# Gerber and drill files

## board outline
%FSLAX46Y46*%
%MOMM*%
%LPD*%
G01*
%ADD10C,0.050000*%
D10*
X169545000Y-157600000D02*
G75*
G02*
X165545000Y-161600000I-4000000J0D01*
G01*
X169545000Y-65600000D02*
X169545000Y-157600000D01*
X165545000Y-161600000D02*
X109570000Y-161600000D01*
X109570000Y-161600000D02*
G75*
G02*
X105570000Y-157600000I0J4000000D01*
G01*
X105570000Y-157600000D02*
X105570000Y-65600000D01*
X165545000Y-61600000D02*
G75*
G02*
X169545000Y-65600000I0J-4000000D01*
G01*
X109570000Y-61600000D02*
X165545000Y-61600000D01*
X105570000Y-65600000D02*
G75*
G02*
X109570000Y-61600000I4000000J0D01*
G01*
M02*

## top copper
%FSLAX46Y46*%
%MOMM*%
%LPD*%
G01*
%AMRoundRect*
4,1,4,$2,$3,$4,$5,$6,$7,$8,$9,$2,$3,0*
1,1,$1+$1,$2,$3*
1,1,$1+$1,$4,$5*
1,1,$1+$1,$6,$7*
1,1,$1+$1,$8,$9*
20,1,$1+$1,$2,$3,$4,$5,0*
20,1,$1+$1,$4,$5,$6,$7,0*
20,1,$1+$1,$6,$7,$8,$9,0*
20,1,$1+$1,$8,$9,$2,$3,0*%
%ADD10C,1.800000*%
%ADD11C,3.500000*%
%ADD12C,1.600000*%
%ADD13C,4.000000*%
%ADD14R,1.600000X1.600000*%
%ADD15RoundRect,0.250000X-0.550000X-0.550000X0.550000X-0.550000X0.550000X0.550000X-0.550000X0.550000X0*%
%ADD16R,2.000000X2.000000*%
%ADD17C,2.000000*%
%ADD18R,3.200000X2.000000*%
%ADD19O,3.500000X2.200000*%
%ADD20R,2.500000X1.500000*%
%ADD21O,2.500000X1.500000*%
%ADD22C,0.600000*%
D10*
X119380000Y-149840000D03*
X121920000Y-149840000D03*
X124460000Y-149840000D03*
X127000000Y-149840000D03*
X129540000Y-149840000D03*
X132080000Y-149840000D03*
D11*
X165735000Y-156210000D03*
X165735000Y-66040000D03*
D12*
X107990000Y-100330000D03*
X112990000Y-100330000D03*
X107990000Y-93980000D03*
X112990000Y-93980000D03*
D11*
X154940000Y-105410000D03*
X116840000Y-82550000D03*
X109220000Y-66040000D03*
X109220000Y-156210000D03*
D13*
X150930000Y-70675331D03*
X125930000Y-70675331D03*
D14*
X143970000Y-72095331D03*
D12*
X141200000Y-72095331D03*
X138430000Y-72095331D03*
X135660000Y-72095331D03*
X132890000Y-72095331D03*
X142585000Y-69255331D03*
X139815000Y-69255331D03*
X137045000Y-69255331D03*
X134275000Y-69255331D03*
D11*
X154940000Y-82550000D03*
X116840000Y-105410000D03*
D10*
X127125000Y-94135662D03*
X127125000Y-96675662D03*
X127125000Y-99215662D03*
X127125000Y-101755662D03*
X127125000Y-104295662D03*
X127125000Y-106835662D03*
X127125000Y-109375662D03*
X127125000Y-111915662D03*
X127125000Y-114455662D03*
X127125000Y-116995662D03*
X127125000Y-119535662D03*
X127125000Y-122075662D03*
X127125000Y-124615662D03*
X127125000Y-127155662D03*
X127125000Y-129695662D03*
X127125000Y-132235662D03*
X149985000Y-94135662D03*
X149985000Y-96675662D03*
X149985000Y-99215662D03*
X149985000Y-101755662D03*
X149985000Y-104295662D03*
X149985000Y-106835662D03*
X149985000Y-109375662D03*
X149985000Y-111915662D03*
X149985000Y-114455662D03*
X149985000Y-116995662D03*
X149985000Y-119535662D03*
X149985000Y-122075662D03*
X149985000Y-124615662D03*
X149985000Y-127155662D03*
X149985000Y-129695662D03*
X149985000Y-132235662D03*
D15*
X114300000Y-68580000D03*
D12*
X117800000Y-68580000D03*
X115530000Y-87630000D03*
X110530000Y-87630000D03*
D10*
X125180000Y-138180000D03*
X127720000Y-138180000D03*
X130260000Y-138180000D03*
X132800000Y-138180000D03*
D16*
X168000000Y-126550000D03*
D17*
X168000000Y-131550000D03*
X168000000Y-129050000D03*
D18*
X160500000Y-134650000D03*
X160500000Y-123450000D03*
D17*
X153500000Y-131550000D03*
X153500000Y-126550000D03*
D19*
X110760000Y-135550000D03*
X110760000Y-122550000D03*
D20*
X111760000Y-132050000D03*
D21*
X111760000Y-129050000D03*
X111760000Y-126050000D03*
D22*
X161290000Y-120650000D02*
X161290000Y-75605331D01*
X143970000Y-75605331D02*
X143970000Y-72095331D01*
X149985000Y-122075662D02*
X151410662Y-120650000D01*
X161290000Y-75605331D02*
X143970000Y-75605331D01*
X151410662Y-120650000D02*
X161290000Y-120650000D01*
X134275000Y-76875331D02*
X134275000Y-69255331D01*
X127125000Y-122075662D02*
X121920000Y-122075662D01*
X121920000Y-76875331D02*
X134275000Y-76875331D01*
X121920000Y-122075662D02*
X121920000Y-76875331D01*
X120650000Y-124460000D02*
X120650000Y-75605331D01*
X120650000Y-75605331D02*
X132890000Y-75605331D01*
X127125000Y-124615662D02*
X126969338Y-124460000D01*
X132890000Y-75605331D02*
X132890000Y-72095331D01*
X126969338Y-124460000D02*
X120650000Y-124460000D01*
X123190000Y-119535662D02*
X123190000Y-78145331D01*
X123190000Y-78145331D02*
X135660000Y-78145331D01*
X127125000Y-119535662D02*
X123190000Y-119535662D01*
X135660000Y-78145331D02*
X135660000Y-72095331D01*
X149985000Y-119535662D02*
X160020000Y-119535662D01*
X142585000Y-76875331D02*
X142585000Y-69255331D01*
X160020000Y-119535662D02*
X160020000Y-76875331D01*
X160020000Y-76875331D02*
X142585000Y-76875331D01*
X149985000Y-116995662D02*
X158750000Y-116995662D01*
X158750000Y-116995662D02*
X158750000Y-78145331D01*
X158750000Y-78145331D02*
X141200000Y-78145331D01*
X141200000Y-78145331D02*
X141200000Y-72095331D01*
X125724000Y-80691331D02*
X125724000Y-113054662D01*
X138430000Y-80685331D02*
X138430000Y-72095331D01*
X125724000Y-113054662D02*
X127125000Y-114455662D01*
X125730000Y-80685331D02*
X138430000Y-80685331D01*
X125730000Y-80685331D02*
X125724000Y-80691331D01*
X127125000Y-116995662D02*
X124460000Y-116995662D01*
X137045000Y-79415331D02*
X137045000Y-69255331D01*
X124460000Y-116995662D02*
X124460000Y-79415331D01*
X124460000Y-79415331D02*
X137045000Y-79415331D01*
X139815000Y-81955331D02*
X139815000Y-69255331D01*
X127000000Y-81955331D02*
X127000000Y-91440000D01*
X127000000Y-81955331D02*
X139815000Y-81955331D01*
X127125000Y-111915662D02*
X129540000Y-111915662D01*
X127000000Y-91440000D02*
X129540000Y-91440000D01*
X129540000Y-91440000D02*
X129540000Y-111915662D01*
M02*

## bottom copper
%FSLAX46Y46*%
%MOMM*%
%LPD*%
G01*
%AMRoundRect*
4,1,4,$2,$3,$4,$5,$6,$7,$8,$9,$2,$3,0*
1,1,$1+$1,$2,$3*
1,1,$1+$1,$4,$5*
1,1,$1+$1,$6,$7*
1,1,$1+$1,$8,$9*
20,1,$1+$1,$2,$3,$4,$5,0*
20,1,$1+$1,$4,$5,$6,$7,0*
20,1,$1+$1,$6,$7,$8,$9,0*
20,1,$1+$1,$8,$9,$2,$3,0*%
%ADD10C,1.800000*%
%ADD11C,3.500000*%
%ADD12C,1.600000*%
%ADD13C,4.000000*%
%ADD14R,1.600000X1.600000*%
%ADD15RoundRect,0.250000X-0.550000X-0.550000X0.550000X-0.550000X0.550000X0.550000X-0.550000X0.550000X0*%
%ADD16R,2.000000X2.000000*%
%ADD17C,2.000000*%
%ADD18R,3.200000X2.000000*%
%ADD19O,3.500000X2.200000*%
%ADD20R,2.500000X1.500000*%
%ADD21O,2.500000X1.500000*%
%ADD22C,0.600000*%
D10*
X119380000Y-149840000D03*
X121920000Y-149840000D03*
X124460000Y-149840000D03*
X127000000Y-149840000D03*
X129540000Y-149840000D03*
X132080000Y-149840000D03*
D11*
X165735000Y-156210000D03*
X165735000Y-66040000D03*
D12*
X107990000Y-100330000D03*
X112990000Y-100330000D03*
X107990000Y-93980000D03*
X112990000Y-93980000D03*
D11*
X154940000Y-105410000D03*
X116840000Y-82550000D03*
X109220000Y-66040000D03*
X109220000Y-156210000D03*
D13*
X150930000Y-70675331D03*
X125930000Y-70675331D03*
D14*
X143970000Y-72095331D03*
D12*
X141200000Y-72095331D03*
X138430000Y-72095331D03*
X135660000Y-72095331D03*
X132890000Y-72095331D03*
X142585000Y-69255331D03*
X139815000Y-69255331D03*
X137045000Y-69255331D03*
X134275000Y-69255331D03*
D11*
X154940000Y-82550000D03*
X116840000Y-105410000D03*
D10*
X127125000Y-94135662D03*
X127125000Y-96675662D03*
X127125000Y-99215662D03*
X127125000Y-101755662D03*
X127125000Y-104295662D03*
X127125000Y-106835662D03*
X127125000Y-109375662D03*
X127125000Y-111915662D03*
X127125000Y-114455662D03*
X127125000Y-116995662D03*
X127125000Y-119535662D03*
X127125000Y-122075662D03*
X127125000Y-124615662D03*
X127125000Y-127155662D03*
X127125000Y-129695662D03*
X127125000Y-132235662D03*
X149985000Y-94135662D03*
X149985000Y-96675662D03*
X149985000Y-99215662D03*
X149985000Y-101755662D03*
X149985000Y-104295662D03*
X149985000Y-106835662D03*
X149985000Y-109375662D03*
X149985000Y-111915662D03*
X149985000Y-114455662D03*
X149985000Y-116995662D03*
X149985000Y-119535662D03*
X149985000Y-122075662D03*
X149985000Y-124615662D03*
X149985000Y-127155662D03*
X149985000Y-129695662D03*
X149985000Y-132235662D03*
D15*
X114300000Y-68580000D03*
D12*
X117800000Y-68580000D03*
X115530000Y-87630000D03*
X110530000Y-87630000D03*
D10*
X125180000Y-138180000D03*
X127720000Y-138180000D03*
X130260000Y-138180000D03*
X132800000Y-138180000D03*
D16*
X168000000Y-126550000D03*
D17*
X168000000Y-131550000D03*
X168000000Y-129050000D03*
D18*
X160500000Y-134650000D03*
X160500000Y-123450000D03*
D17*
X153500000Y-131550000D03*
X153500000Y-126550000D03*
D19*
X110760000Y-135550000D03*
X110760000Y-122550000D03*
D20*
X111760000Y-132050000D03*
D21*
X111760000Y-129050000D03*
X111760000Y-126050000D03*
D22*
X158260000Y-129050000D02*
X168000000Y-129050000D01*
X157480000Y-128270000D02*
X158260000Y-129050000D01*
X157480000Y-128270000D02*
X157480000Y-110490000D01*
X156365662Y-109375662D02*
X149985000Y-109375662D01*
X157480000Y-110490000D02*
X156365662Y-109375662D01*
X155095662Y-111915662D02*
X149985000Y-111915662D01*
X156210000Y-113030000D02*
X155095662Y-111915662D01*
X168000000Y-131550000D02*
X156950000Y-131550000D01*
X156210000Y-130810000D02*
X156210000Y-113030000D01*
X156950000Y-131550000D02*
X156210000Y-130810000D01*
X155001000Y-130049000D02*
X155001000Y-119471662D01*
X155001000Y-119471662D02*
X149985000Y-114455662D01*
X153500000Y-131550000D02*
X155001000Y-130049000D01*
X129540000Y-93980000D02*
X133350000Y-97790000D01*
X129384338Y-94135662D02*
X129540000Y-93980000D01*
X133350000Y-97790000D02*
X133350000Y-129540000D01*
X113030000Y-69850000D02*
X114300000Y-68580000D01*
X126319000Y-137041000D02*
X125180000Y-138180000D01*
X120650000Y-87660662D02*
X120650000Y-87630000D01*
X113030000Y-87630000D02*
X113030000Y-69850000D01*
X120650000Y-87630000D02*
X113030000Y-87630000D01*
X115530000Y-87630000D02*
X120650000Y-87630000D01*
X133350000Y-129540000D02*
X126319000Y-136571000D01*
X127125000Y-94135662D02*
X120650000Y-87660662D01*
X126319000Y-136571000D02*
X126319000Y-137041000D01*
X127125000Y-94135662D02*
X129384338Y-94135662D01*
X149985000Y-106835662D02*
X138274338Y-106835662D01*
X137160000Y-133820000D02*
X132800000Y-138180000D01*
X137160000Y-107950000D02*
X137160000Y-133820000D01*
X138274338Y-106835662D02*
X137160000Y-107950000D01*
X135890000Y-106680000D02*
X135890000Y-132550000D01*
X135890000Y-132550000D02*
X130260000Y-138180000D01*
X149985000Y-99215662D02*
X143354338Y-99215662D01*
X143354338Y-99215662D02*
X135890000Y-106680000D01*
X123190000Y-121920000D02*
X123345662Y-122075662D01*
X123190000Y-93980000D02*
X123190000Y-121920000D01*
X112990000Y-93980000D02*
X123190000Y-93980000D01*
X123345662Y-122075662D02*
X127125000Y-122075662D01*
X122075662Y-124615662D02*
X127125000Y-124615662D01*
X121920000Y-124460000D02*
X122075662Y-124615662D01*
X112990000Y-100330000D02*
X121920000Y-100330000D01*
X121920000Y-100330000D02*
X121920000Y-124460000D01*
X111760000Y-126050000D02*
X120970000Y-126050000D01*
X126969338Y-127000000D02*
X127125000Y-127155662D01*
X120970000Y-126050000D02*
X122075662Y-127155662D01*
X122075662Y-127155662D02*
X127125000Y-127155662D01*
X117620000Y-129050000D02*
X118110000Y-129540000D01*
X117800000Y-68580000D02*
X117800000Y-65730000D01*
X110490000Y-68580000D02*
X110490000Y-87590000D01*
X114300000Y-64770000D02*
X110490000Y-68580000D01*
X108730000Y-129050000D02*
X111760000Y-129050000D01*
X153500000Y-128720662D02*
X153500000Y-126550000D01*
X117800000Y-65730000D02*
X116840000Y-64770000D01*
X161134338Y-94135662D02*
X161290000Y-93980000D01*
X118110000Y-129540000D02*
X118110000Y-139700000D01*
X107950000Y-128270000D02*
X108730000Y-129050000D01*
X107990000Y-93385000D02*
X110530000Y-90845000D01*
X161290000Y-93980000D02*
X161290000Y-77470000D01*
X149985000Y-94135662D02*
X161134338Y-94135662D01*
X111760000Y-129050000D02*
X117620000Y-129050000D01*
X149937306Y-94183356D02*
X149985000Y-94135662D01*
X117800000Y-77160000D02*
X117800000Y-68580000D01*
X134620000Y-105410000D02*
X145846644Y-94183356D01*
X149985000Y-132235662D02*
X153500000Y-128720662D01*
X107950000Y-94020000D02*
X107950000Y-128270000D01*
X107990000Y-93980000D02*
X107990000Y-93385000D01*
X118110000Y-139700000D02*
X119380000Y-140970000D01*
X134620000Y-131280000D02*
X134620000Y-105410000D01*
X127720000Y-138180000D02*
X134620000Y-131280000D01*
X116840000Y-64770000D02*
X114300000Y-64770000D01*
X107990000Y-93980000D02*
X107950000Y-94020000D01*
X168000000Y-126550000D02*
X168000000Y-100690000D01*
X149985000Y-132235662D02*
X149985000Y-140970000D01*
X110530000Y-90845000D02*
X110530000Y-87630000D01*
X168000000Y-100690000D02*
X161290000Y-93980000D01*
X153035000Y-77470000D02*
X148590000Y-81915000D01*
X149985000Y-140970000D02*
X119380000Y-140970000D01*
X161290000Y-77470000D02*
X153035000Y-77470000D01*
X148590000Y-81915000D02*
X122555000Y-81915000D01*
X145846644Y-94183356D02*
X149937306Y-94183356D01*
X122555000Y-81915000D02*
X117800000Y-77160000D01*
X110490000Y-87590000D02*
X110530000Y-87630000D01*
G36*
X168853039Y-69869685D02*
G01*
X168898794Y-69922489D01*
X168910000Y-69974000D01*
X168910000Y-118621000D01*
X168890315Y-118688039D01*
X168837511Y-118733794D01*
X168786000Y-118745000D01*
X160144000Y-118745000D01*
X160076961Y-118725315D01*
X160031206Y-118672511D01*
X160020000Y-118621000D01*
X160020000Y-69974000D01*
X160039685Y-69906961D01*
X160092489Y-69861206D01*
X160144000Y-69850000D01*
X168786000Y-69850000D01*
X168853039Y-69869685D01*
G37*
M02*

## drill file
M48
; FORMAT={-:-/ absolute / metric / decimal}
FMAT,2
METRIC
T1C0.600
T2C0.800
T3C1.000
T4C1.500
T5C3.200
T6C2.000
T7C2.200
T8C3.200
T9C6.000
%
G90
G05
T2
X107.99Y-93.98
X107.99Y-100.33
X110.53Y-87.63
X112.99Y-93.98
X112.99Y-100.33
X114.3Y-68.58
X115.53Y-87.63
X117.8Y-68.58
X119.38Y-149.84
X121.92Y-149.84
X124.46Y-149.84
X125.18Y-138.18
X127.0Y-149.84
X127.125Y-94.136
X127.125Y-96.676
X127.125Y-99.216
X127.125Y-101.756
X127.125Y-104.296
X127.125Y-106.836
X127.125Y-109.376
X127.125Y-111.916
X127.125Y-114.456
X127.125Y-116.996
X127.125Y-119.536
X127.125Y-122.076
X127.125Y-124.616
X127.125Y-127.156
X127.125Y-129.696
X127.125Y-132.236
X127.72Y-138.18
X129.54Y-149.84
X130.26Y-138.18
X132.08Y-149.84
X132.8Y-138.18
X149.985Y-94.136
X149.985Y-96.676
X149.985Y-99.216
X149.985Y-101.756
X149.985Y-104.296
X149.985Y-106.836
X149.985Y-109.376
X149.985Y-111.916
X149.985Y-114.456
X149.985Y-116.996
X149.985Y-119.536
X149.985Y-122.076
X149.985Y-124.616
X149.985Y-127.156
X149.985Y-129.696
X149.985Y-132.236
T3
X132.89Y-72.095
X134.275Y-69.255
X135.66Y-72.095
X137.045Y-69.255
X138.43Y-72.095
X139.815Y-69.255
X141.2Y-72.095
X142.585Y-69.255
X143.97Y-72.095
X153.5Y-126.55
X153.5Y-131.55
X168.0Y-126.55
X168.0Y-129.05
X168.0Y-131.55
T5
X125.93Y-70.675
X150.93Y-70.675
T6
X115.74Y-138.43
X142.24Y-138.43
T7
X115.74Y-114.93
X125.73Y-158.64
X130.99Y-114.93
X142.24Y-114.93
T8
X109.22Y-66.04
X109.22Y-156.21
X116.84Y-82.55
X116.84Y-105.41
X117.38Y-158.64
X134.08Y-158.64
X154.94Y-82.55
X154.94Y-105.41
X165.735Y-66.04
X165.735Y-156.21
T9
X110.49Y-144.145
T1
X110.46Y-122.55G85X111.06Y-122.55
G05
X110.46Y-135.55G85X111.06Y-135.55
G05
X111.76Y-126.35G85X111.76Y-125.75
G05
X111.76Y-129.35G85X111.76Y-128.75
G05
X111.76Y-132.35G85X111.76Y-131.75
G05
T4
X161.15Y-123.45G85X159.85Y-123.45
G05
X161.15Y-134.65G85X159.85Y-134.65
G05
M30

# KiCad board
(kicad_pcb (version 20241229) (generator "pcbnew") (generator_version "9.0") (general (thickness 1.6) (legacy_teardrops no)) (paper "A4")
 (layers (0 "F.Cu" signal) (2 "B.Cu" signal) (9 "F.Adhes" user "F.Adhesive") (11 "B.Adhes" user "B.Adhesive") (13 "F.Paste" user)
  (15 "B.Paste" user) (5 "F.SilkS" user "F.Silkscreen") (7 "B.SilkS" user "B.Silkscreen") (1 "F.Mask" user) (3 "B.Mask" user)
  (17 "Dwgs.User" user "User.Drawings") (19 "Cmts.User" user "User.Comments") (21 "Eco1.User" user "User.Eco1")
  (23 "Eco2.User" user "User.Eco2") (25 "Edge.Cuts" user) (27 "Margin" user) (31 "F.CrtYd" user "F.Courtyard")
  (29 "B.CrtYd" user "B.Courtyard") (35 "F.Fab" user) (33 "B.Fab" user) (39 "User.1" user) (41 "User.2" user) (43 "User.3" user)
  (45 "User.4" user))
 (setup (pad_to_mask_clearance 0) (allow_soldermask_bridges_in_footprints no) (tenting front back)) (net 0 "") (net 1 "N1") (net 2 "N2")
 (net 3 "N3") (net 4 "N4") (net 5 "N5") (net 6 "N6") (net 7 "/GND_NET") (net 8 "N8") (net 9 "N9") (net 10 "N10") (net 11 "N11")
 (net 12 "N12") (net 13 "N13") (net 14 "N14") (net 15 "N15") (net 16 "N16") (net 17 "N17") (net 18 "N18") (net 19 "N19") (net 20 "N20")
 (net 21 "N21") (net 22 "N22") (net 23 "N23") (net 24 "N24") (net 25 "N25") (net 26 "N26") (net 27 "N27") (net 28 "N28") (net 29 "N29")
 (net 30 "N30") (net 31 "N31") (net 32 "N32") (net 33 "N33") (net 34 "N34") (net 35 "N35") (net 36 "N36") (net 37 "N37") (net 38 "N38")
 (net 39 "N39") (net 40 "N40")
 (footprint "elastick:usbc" (layer "F.Cu") (at 125.73 148.64)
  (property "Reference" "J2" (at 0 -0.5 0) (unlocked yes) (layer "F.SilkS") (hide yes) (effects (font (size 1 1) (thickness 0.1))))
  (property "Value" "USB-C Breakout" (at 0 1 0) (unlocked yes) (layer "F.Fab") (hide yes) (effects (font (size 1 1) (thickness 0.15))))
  (pad "" np_thru_hole circle (at -8.35 10) (size 3.2 3.2) (drill 3.2) (layers "*.Cu" "*.Mask"))
  (pad "" np_thru_hole circle (at 0 10) (size 2.2 2.2) (drill 2.2) (layers "*.Cu" "*.Mask"))
  (pad "" np_thru_hole circle (at 8.35 10) (size 3.2 3.2) (drill 3.2) (layers "*.Cu" "*.Mask"))
  (pad "1" thru_hole circle (at -6.35 1.2) (size 1.8 1.8) (drill 0.8) (layers "*.Cu" "*.Mask") (remove_unused_layers no) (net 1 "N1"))
  (pad "2" thru_hole circle (at -3.81 1.2) (size 1.8 1.8) (drill 0.8) (layers "*.Cu" "*.Mask") (remove_unused_layers no) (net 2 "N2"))
  (pad "3" thru_hole circle (at -1.27 1.2) (size 1.8 1.8) (drill 0.8) (layers "*.Cu" "*.Mask") (remove_unused_layers no) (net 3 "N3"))
  (pad "4" thru_hole circle (at 1.27 1.2) (size 1.8 1.8) (drill 0.8) (layers "*.Cu" "*.Mask") (remove_unused_layers no) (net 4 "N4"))
  (pad "5" thru_hole circle (at 3.81 1.2) (size 1.8 1.8) (drill 0.8) (layers "*.Cu" "*.Mask") (remove_unused_layers no) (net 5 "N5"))
  (pad "6" thru_hole circle (at 6.35 1.2) (size 1.8 1.8) (drill 0.8) (layers "*.Cu" "*.Mask") (remove_unused_layers no) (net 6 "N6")))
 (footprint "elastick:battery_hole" (layer "F.Cu") (at 165.735 156.21)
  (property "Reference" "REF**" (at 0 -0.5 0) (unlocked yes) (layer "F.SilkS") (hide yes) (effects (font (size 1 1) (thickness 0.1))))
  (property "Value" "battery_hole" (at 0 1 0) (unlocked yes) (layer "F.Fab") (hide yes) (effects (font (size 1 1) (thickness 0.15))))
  (pad "" np_thru_hole circle (at 0 0) (size 3.5 3.5) (drill 3.2) (layers "*.Cu" "*.Mask")))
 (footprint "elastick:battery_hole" (layer "F.Cu") (at 165.735 66.04)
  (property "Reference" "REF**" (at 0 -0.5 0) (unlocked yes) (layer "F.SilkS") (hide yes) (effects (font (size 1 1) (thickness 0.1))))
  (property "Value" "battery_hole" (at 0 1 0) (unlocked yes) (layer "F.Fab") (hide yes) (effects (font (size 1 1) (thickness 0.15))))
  (pad "" np_thru_hole circle (at 0 0) (size 3.5 3.5) (drill 3.2) (layers "*.Cu" "*.Mask")))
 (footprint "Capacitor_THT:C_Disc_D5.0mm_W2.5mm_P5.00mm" (layer "F.Cu") (at 107.99 100.33)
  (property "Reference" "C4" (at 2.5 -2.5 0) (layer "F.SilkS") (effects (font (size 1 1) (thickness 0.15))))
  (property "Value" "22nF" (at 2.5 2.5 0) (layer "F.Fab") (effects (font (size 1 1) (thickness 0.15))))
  (pad "1" thru_hole circle (at 0 0) (size 1.6 1.6) (drill 0.8) (layers "*.Cu" "*.Mask") (remove_unused_layers no) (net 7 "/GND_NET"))
  (pad "2" thru_hole circle (at 5 0) (size 1.6 1.6) (drill 0.8) (layers "*.Cu" "*.Mask") (remove_unused_layers no) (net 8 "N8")))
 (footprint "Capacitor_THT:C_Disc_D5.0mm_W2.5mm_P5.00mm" (layer "F.Cu") (at 107.99 93.98)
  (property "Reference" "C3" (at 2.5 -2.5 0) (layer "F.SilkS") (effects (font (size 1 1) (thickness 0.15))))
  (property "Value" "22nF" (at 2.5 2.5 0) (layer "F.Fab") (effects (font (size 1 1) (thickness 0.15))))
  (pad "1" thru_hole circle (at 0 0) (size 1.6 1.6) (drill 0.8) (layers "*.Cu" "*.Mask") (remove_unused_layers no) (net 7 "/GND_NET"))
  (pad "2" thru_hole circle (at 5 0) (size 1.6 1.6) (drill 0.8) (layers "*.Cu" "*.Mask") (remove_unused_layers no) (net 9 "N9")))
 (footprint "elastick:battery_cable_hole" (layer "F.Cu") (at 110.49 144.145)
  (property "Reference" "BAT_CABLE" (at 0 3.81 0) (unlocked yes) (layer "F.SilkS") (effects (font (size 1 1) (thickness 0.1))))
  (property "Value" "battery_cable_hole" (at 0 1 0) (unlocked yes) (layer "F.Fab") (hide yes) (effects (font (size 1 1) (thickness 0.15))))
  (pad "" np_thru_hole circle (at 0 0) (size 6 6) (drill 6) (layers "*.Cu" "*.Mask")))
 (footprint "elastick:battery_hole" (layer "F.Cu") (at 154.94 105.41)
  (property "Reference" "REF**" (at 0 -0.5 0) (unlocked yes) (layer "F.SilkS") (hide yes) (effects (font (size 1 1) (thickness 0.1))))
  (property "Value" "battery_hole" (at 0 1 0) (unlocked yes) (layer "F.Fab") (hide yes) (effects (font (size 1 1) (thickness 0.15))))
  (pad "" np_thru_hole circle (at 0 0) (size 3.5 3.5) (drill 3.2) (layers "*.Cu" "*.Mask")))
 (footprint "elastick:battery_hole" (layer "F.Cu") (at 116.84 82.55)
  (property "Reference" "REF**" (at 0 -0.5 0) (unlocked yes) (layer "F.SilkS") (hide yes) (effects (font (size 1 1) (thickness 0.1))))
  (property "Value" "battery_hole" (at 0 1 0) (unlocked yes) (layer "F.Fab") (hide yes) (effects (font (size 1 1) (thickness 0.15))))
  (pad "" np_thru_hole circle (at 0 0) (size 3.5 3.5) (drill 3.2) (layers "*.Cu" "*.Mask")))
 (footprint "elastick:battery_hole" (layer "F.Cu") (at 109.22 66.04)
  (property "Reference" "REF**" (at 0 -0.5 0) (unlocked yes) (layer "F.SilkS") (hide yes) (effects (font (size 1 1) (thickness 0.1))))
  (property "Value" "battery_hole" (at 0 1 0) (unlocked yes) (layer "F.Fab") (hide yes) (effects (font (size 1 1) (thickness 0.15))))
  (pad "" np_thru_hole circle (at 0 0) (size 3.5 3.5) (drill 3.2) (layers "*.Cu" "*.Mask")))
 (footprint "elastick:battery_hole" (layer "F.Cu") (at 109.22 156.21)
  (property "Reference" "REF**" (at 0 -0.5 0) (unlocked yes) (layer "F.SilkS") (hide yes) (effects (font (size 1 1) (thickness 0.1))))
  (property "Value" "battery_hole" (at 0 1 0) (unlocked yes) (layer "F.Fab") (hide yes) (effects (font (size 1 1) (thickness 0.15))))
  (pad "" np_thru_hole circle (at 0 0) (size 3.5 3.5) (drill 3.2) (layers "*.Cu" "*.Mask")))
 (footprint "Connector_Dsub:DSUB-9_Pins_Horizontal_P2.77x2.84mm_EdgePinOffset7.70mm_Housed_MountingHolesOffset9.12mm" (layer "F.Cu")
  (at 143.97 72.095331 180)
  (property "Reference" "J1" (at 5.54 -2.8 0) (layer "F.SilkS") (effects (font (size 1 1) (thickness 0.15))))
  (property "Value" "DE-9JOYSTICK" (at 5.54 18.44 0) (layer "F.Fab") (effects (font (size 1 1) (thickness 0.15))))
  (pad "0" thru_hole circle (at -6.96 1.42 180) (size 4 4) (drill 3.2) (layers "*.Cu" "*.Mask") (remove_unused_layers no) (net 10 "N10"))
  (pad "0" thru_hole circle (at 18.04 1.42 180) (size 4 4) (drill 3.2) (layers "*.Cu" "*.Mask") (remove_unused_layers no) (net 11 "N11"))
  (pad "1" thru_hole rect (at 0 0 180) (size 1.6 1.6) (drill 1) (layers "*.Cu" "*.Mask") (remove_unused_layers no) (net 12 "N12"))
  (pad "2" thru_hole circle (at 2.77 0 180) (size 1.6 1.6) (drill 1) (layers "*.Cu" "*.Mask") (remove_unused_layers no) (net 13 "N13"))
  (pad "3" thru_hole circle (at 5.54 0 180) (size 1.6 1.6) (drill 1) (layers "*.Cu" "*.Mask") (remove_unused_layers no) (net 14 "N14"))
  (pad "4" thru_hole circle (at 8.31 0 180) (size 1.6 1.6) (drill 1) (layers "*.Cu" "*.Mask") (remove_unused_layers no) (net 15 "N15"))
  (pad "5" thru_hole circle (at 11.08 0 180) (size 1.6 1.6) (drill 1) (layers "*.Cu" "*.Mask") (remove_unused_layers no) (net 8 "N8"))
  (pad "6" thru_hole circle (at 1.385 2.84 180) (size 1.6 1.6) (drill 1) (layers "*.Cu" "*.Mask") (remove_unused_layers no) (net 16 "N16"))
  (pad "7" thru_hole circle (at 4.155 2.84 180) (size 1.6 1.6) (drill 1) (layers "*.Cu" "*.Mask") (remove_unused_layers no) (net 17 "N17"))
  (pad "8" thru_hole circle (at 6.925 2.84 180) (size 1.6 1.6) (drill 1) (layers "*.Cu" "*.Mask") (remove_unused_layers no) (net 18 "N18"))
  (pad "9" thru_hole circle (at 9.695 2.84 180) (size 1.6 1.6) (drill 1) (layers "*.Cu" "*.Mask") (remove_unused_layers no) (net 9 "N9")))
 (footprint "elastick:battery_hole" (layer "F.Cu") (at 154.94 82.55)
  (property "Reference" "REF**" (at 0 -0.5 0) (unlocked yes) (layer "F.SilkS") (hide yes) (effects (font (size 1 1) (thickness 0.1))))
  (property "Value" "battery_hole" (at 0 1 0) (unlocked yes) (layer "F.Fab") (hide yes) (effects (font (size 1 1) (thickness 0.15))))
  (pad "" np_thru_hole circle (at 0 0) (size 3.5 3.5) (drill 3.2) (layers "*.Cu" "*.Mask")))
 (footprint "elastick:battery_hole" (layer "F.Cu") (at 116.84 105.41)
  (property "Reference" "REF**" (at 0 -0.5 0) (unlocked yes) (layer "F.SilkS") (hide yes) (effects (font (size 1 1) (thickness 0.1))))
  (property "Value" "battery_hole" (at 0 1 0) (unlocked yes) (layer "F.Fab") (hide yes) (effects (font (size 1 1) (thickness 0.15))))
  (pad "" np_thru_hole circle (at 0 0) (size 3.5 3.5) (drill 3.2) (layers "*.Cu" "*.Mask")))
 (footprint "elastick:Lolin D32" (layer "F.Cu") (at 134.745 134.775662)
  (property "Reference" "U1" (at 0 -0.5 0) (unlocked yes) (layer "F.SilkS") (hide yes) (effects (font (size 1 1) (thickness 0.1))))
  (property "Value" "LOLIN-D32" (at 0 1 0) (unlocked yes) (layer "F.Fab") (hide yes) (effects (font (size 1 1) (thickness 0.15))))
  (pad "1" thru_hole circle (at -7.62 -40.64) (size 1.8 1.8) (drill 0.8) (layers "*.Cu" "*.Mask") (remove_unused_layers no) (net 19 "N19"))
  (pad "2" thru_hole circle (at -7.62 -38.1) (size 1.8 1.8) (drill 0.8) (layers "*.Cu" "*.Mask") (remove_unused_layers no) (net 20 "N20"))
  (pad "3" thru_hole circle (at -7.62 -35.56) (size 1.8 1.8) (drill 0.8) (layers "*.Cu" "*.Mask") (remove_unused_layers no) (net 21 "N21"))
  (pad "4" thru_hole circle (at -7.62 -33.02) (size 1.8 1.8) (drill 0.8) (layers "*.Cu" "*.Mask") (remove_unused_layers no) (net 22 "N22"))
  (pad "5" thru_hole circle (at -7.62 -30.48) (size 1.8 1.8) (drill 0.8) (layers "*.Cu" "*.Mask") (remove_unused_layers no) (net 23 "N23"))
  (pad "6" thru_hole circle (at -7.62 -27.94) (size 1.8 1.8) (drill 0.8) (layers "*.Cu" "*.Mask") (remove_unused_layers no) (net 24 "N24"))
  (pad "7" thru_hole circle (at -7.62 -25.4) (size 1.8 1.8) (drill 0.8) (layers "*.Cu" "*.Mask") (remove_unused_layers no) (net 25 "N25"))
  (pad "8" thru_hole circle (at -7.62 -22.86) (size 1.8 1.8) (drill 0.8) (layers "*.Cu" "*.Mask") (remove_unused_layers no) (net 17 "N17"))
  (pad "9" thru_hole circle (at -7.62 -20.32) (size 1.8 1.8) (drill 0.8) (layers "*.Cu" "*.Mask") (remove_unused_layers no) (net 14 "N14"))
  (pad "10" thru_hole circle (at -7.62 -17.78) (size 1.8 1.8) (drill 0.8) (layers "*.Cu" "*.Mask") (remove_unused_layers no) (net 18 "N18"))
  (pad "11" thru_hole circle (at -7.62 -15.24) (size 1.8 1.8) (drill 0.8) (layers "*.Cu" "*.Mask") (remove_unused_layers no) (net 15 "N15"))
  (pad "12" thru_hole circle (at -7.62 -12.7) (size 1.8 1.8) (drill 0.8) (layers "*.Cu" "*.Mask") (remove_unused_layers no) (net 9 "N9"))
  (pad "13" thru_hole circle (at -7.62 -10.16) (size 1.8 1.8) (drill 0.8) (layers "*.Cu" "*.Mask") (remove_unused_layers no) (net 8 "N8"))
  (pad "14" thru_hole circle (at -7.62 -7.62) (size 1.8 1.8) (drill 0.8) (layers "*.Cu" "*.Mask") (remove_unused_layers no) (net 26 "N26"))
  (pad "15" thru_hole circle (at -7.62 -5.08) (size 1.8 1.8) (drill 0.8) (layers "*.Cu" "*.Mask") (remove_unused_layers no) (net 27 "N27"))
  (pad "16" thru_hole circle (at -7.62 -2.54) (size 1.8 1.8) (drill 0.8) (layers "*.Cu" "*.Mask") (remove_unused_layers no) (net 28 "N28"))
  (pad "17" thru_hole circle (at 15.24 -40.64) (size 1.8 1.8) (drill 0.8) (layers "*.Cu" "*.Mask") (remove_unused_layers no)
   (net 7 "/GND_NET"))
  (pad "18" thru_hole circle (at 15.24 -38.1) (size 1.8 1.8) (drill 0.8) (layers "*.Cu" "*.Mask") (remove_unused_layers no) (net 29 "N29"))
  (pad "19" thru_hole circle (at 15.24 -35.56) (size 1.8 1.8) (drill 0.8) (layers "*.Cu" "*.Mask") (remove_unused_layers no) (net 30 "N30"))
  (pad "20" thru_hole circle (at 15.24 -33.02) (size 1.8 1.8) (drill 0.8) (layers "*.Cu" "*.Mask") (remove_unused_layers no) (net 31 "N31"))
  (pad "21" thru_hole circle (at 15.24 -30.48) (size 1.8 1.8) (drill 0.8) (layers "*.Cu" "*.Mask") (remove_unused_layers no) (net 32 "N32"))
  (pad "22" thru_hole circle (at 15.24 -27.94) (size 1.8 1.8) (drill 0.8) (layers "*.Cu" "*.Mask") (remove_unused_layers no) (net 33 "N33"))
  (pad "23" thru_hole circle (at 15.24 -25.4) (size 1.8 1.8) (drill 0.8) (layers "*.Cu" "*.Mask") (remove_unused_layers no) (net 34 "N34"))
  (pad "24" thru_hole circle (at 15.24 -22.86) (size 1.8 1.8) (drill 0.8) (layers "*.Cu" "*.Mask") (remove_unused_layers no) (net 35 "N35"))
  (pad "25" thru_hole circle (at 15.24 -20.32) (size 1.8 1.8) (drill 0.8) (layers "*.Cu" "*.Mask") (remove_unused_layers no) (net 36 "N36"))
  (pad "26" thru_hole circle (at 15.24 -17.78) (size 1.8 1.8) (drill 0.8) (layers "*.Cu" "*.Mask") (remove_unused_layers no) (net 13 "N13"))
  (pad "27" thru_hole circle (at 15.24 -15.24) (size 1.8 1.8) (drill 0.8) (layers "*.Cu" "*.Mask") (remove_unused_layers no) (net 16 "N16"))
  (pad "28" thru_hole circle (at 15.24 -12.7) (size 1.8 1.8) (drill 0.8) (layers "*.Cu" "*.Mask") (remove_unused_layers no) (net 12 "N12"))
  (pad "29" thru_hole circle (at 15.24 -10.16) (size 1.8 1.8) (drill 0.8) (layers "*.Cu" "*.Mask") (remove_unused_layers no) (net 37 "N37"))
  (pad "30" thru_hole circle (at 15.24 -7.62) (size 1.8 1.8) (drill 0.8) (layers "*.Cu" "*.Mask") (remove_unused_layers no) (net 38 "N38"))
  (pad "31" thru_hole circle (at 15.24 -5.08) (size 1.8 1.8) (drill 0.8) (layers "*.Cu" "*.Mask") (remove_unused_layers no) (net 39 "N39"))
  (pad "32" thru_hole circle (at 15.24 -2.54) (size 1.8 1.8) (drill 0.8) (layers "*.Cu" "*.Mask") (remove_unused_layers no)
   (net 7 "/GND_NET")))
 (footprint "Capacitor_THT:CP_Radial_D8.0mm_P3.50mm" (layer "F.Cu") (at 114.3 68.58)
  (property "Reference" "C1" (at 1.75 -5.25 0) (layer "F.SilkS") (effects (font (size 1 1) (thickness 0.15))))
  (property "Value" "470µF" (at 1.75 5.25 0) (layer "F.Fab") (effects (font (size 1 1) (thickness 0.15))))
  (pad "1" thru_hole roundrect (at 0 0) (size 1.6 1.6) (drill 0.8) (layers "*.Cu" "*.Mask") (remove_unused_layers no)
   (roundrect_rratio 0.15625) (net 19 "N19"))
  (pad "2" thru_hole circle (at 3.5 0) (size 1.6 1.6) (drill 0.8) (layers "*.Cu" "*.Mask") (remove_unused_layers no) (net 7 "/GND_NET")))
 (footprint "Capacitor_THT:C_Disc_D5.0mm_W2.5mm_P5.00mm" (layer "F.Cu") (at 115.53 87.63 180)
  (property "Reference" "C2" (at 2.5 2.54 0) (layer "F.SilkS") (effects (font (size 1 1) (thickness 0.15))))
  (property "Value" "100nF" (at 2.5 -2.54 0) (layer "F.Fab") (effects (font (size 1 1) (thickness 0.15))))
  (pad "1" thru_hole circle (at 0 0 180) (size 1.6 1.6) (drill 0.8) (layers "*.Cu" "*.Mask") (remove_unused_layers no) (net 19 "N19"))
  (pad "2" thru_hole circle (at 5 0 180) (size 1.6 1.6) (drill 0.8) (layers "*.Cu" "*.Mask") (remove_unused_layers no) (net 7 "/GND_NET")))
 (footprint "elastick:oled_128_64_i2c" (layer "B.Cu") (at 128.99 138.18)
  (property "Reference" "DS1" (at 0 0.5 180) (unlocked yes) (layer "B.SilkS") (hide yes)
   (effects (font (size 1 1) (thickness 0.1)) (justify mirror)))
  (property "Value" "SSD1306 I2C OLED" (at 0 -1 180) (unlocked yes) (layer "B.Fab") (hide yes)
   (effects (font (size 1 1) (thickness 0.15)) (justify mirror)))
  (pad "" np_thru_hole circle (at -13.25 -23.25) (size 2.2 2.2) (drill 2.2) (layers "*.Cu" "*.Mask"))
  (pad "" np_thru_hole circle (at -13.25 0.25) (size 2 2) (drill 2) (layers "*.Cu" "*.Mask"))
  (pad "" np_thru_hole circle (at 2 -23.25) (size 2.2 2.2) (drill 2.2) (layers "*.Cu" "*.Mask"))
  (pad "" np_thru_hole circle (at 13.25 -23.25) (size 2.2 2.2) (drill 2.2) (layers "*.Cu" "*.Mask"))
  (pad "" np_thru_hole circle (at 13.25 0.25) (size 2 2) (drill 2) (layers "*.Cu" "*.Mask"))
  (pad "1" thru_hole circle (at -3.81 0) (size 1.8 1.8) (drill 0.8) (layers "*.Cu" "*.Mask") (remove_unused_layers no) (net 19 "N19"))
  (pad "2" thru_hole circle (at -1.27 0) (size 1.8 1.8) (drill 0.8) (layers "*.Cu" "*.Mask") (remove_unused_layers no) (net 7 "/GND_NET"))
  (pad "3" thru_hole circle (at 1.27 0) (size 1.8 1.8) (drill 0.8) (layers "*.Cu" "*.Mask") (remove_unused_layers no) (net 30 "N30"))
  (pad "4" thru_hole circle (at 3.81 0) (size 1.8 1.8) (drill 0.8) (layers "*.Cu" "*.Mask") (remove_unused_layers no) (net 33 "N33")))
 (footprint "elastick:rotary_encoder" (layer "B.Cu") (at 168 126.55 180)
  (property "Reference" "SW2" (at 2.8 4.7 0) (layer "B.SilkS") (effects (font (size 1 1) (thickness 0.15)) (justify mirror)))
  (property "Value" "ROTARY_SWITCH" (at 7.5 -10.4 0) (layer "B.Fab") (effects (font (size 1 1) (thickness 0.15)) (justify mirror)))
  (pad "A" thru_hole rect (at 0 0 180) (size 2 2) (drill 1) (layers "*.Cu" "*.Mask") (remove_unused_layers no) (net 7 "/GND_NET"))
  (pad "B" thru_hole circle (at 0 -5 180) (size 2 2) (drill 1) (layers "*.Cu" "*.Mask") (remove_unused_layers no) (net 35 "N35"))
  (pad "C" thru_hole circle (at 0 -2.5 180) (size 2 2) (drill 1) (layers "*.Cu" "*.Mask") (remove_unused_layers no) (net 34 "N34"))
  (pad "MP" thru_hole rect (at 7.5 -8.1 180) (size 3.2 2) (drill oval 2.8 1.5) (layers "*.Cu" "*.Mask") (remove_unused_layers no))
  (pad "MP" thru_hole rect (at 7.5 3.1 180) (size 3.2 2) (drill oval 2.8 1.5) (layers "*.Cu" "*.Mask") (remove_unused_layers no))
  (pad "S1" thru_hole circle (at 14.5 -5 180) (size 2 2) (drill 1) (layers "*.Cu" "*.Mask") (remove_unused_layers no) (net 36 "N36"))
  (pad "S2" thru_hole circle (at 14.5 0 180) (size 2 2) (drill 1) (layers "*.Cu" "*.Mask") (remove_unused_layers no) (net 7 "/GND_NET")))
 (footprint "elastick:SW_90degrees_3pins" (layer "B.Cu") (at 111.76 132.05 90)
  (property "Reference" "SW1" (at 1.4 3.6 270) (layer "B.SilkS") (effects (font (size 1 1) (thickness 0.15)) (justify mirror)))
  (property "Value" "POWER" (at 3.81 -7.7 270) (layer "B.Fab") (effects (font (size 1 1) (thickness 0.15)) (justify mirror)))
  (pad "" thru_hole oval (at -3.5 -1 90) (size 2.2 3.5) (drill oval 0.6 1.2) (layers "*.Cu" "*.Mask") (remove_unused_layers no))
  (pad "" thru_hole oval (at 9.5 -1 90) (size 2.2 3.5) (drill oval 0.6 1.2) (layers "*.Cu" "*.Mask") (remove_unused_layers no))
  (pad "1" thru_hole rect (at 0 0 90) (size 1.5 2.5) (drill oval 1.2 0.6) (layers "*.Cu" "*.Mask") (remove_unused_layers no) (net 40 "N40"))
  (pad "2" thru_hole oval (at 3 0 90) (size 1.5 2.5) (drill oval 1.2 0.6) (layers "*.Cu" "*.Mask") (remove_unused_layers no)
   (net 7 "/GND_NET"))
  (pad "3" thru_hole oval (at 6 0 90) (size 1.5 2.5) (drill oval 1.2 0.6) (layers "*.Cu" "*.Mask") (remove_unused_layers no) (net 26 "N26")))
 (gr_arc (start 169.545 157.6) (mid 168.373427 160.428427) (end 165.545 161.6) (stroke (width 0.05) (type default)) (layer "Edge.Cuts"))
 (gr_line (start 169.545 65.6) (end 169.545 157.6) (stroke (width 0.05) (type default)) (layer "Edge.Cuts"))
 (gr_line (start 165.545 161.6) (end 109.57 161.6) (stroke (width 0.05) (type default)) (layer "Edge.Cuts"))
 (gr_arc (start 109.57 161.6) (mid 106.741573 160.428427) (end 105.57 157.6) (stroke (width 0.05) (type default)) (layer "Edge.Cuts"))
 (gr_line (start 105.57 157.6) (end 105.57 65.6) (stroke (width 0.05) (type default)) (layer "Edge.Cuts"))
 (gr_arc (start 165.545 61.6) (mid 168.373427 62.771573) (end 169.545 65.6) (stroke (width 0.05) (type default)) (layer "Edge.Cuts"))
 (gr_line (start 109.57 61.6) (end 165.545 61.6) (stroke (width 0.05) (type default)) (layer "Edge.Cuts"))
 (gr_arc (start 105.57 65.6) (mid 106.741573 62.771573) (end 109.57 61.6) (stroke (width 0.05) (type default)) (layer "Edge.Cuts"))
 (segment (start 158.26 129.05) (end 168 129.05) (width 0.6) (layer "B.Cu") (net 34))
 (segment (start 157.48 128.27) (end 158.26 129.05) (width 0.6) (layer "B.Cu") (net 34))
 (segment (start 157.48 128.27) (end 157.48 110.49) (width 0.6) (layer "B.Cu") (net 34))
 (segment (start 156.365662 109.375662) (end 149.985 109.375662) (width 0.6) (layer "B.Cu") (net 34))
 (segment (start 157.48 110.49) (end 156.365662 109.375662) (width 0.6) (layer "B.Cu") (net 34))
 (segment (start 155.095662 111.915662) (end 149.985 111.915662) (width 0.6) (layer "B.Cu") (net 35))
 (segment (start 156.21 113.03) (end 155.095662 111.915662) (width 0.6) (layer "B.Cu") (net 35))
 (segment (start 168 131.55) (end 156.95 131.55) (width 0.6) (layer "B.Cu") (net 35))
 (segment (start 156.21 130.81) (end 156.21 113.03) (width 0.6) (layer "B.Cu") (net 35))
 (segment (start 156.95 131.55) (end 156.21 130.81) (width 0.6) (layer "B.Cu") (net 35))
 (segment (start 155.001 130.049) (end 155.001 119.471662) (width 0.6) (layer "B.Cu") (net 36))
 (segment (start 155.001 119.471662) (end 149.985 114.455662) (width 0.6) (layer "B.Cu") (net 36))
 (segment (start 153.5 131.55) (end 155.001 130.049) (width 0.6) (layer "B.Cu") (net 36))
 (segment (start 129.54 93.98) (end 133.35 97.79) (width 0.6) (layer "B.Cu") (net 19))
 (segment (start 129.384338 94.135662) (end 129.54 93.98) (width 0.6) (layer "B.Cu") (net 19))
 (segment (start 133.35 97.79) (end 133.35 129.54) (width 0.6) (layer "B.Cu") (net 19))
 (segment (start 113.03 69.85) (end 114.3 68.58) (width 0.6) (layer "B.Cu") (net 19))
 (segment (start 126.319 137.041) (end 125.18 138.18) (width 0.6) (layer "B.Cu") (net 19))
 (segment (start 120.65 87.660662) (end 120.65 87.63) (width 0.6) (layer "B.Cu") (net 19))
 (segment (start 113.03 87.63) (end 113.03 69.85) (width 0.6) (layer "B.Cu") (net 19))
 (segment (start 120.65 87.63) (end 113.03 87.63) (width 0.6) (layer "B.Cu") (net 19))
 (segment (start 115.53 87.63) (end 120.65 87.63) (width 0.6) (layer "B.Cu") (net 19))
 (segment (start 133.35 129.54) (end 126.319 136.571) (width 0.6) (layer "B.Cu") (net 19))
 (segment (start 127.125 94.135662) (end 120.65 87.660662) (width 0.6) (layer "B.Cu") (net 19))
 (segment (start 126.319 136.571) (end 126.319 137.041) (width 0.6) (layer "B.Cu") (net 19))
 (segment (start 127.125 94.135662) (end 129.384338 94.135662) (width 0.6) (layer "B.Cu") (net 19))
 (segment (start 149.985 106.835662) (end 138.274338 106.835662) (width 0.6) (layer "B.Cu") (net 33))
 (segment (start 137.16 133.82) (end 132.8 138.18) (width 0.6) (layer "B.Cu") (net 33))
 (segment (start 137.16 107.95) (end 137.16 133.82) (width 0.6) (layer "B.Cu") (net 33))
 (segment (start 138.274338 106.835662) (end 137.16 107.95) (width 0.6) (layer "B.Cu") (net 33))
 (segment (start 135.89 106.68) (end 135.89 132.55) (width 0.6) (layer "B.Cu") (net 30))
 (segment (start 135.89 132.55) (end 130.26 138.18) (width 0.6) (layer "B.Cu") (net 30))
 (segment (start 149.985 99.215662) (end 143.354338 99.215662) (width 0.6) (layer "B.Cu") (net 30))
 (segment (start 143.354338 99.215662) (end 135.89 106.68) (width 0.6) (layer "B.Cu") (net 30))
 (segment (start 161.29 120.65) (end 161.29 75.605331) (width 0.6) (layer "F.Cu") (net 12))
 (segment (start 143.97 75.605331) (end 143.97 72.095331) (width 0.6) (layer "F.Cu") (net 12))
 (segment (start 149.985 122.075662) (end 151.410662 120.65) (width 0.6) (layer "F.Cu") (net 12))
 (segment (start 161.29 75.605331) (end 143.97 75.605331) (width 0.6) (layer "F.Cu") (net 12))
 (segment (start 151.410662 120.65) (end 161.29 120.65) (width 0.6) (layer "F.Cu") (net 12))
 (segment (start 134.275 76.875331) (end 134.275 69.255331) (width 0.6) (layer "F.Cu") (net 9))
 (segment (start 127.125 122.075662) (end 121.92 122.075662) (width 0.6) (layer "F.Cu") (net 9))
 (segment (start 121.92 76.875331) (end 134.275 76.875331) (width 0.6) (layer "F.Cu") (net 9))
 (segment (start 121.92 122.075662) (end 121.92 76.875331) (width 0.6) (layer "F.Cu") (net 9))
 (segment (start 123.19 121.92) (end 123.345662 122.075662) (width 0.6) (layer "B.Cu") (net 9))
 (segment (start 123.19 93.98) (end 123.19 121.92) (width 0.6) (layer "B.Cu") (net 9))
 (segment (start 112.99 93.98) (end 123.19 93.98) (width 0.6) (layer "B.Cu") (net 9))
 (segment (start 123.345662 122.075662) (end 127.125 122.075662) (width 0.6) (layer "B.Cu") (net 9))
 (segment (start 120.65 124.46) (end 120.65 75.605331) (width 0.6) (layer "F.Cu") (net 8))
 (segment (start 120.65 75.605331) (end 132.89 75.605331) (width 0.6) (layer "F.Cu") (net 8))
 (segment (start 127.125 124.615662) (end 126.969338 124.46) (width 0.6) (layer "F.Cu") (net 8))
 (segment (start 132.89 75.605331) (end 132.89 72.095331) (width 0.6) (layer "F.Cu") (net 8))
 (segment (start 126.969338 124.46) (end 120.65 124.46) (width 0.6) (layer "F.Cu") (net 8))
 (segment (start 122.075662 124.615662) (end 127.125 124.615662) (width 0.6) (layer "B.Cu") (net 8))
 (segment (start 121.92 124.46) (end 122.075662 124.615662) (width 0.6) (layer "B.Cu") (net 8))
 (segment (start 112.99 100.33) (end 121.92 100.33) (width 0.6) (layer "B.Cu") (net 8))
 (segment (start 121.92 100.33) (end 121.92 124.46) (width 0.6) (layer "B.Cu") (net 8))
 (segment (start 123.19 119.535662) (end 123.19 78.145331) (width 0.6) (layer "F.Cu") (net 15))
 (segment (start 123.19 78.145331) (end 135.66 78.145331) (width 0.6) (layer "F.Cu") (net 15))
 (segment (start 127.125 119.535662) (end 123.19 119.535662) (width 0.6) (layer "F.Cu") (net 15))
 (segment (start 135.66 78.145331) (end 135.66 72.095331) (width 0.6) (layer "F.Cu") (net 15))
 (segment (start 149.985 119.535662) (end 160.02 119.535662) (width 0.6) (layer "F.Cu") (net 16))
 (segment (start 142.585 76.875331) (end 142.585 69.255331) (width 0.6) (layer "F.Cu") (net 16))
 (segment (start 160.02 119.535662) (end 160.02 76.875331) (width 0.6) (layer "F.Cu") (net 16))
 (segment (start 160.02 76.875331) (end 142.585 76.875331) (width 0.6) (layer "F.Cu") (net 16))
 (segment (start 149.985 116.995662) (end 158.75 116.995662) (width 0.6) (layer "F.Cu") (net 13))
 (segment (start 158.75 116.995662) (end 158.75 78.145331) (width 0.6) (layer "F.Cu") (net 13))
 (segment (start 158.75 78.145331) (end 141.2 78.145331) (width 0.6) (layer "F.Cu") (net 13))
 (segment (start 141.2 78.145331) (end 141.2 72.095331) (width 0.6) (layer "F.Cu") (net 13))
 (segment (start 125.724 80.691331) (end 125.724 113.054662) (width 0.6) (layer "F.Cu") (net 14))
 (segment (start 138.43 80.685331) (end 138.43 72.095331) (width 0.6) (layer "F.Cu") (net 14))
 (segment (start 125.724 113.054662) (end 127.125 114.455662) (width 0.6) (layer "F.Cu") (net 14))
 (segment (start 125.73 80.685331) (end 138.43 80.685331) (width 0.6) (layer "F.Cu") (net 14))
 (segment (start 125.73 80.685331) (end 125.724 80.691331) (width 0.6) (layer "F.Cu") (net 14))
 (segment (start 127.125 116.995662) (end 124.46 116.995662) (width 0.6) (layer "F.Cu") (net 18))
 (segment (start 137.045 79.415331) (end 137.045 69.255331) (width 0.6) (layer "F.Cu") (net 18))
 (segment (start 124.46 116.995662) (end 124.46 79.415331) (width 0.6) (layer "F.Cu") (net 18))
 (segment (start 124.46 79.415331) (end 137.045 79.415331) (width 0.6) (layer "F.Cu") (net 18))
 (segment (start 139.815 81.955331) (end 139.815 69.255331) (width 0.6) (layer "F.Cu") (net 17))
 (segment (start 127 81.955331) (end 127 91.44) (width 0.6) (layer "F.Cu") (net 17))
 (segment (start 127 81.955331) (end 139.815 81.955331) (width 0.6) (layer "F.Cu") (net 17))
 (segment (start 127.125 111.915662) (end 129.54 111.915662) (width 0.6) (layer "F.Cu") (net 17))
 (segment (start 127 91.44) (end 129.54 91.44) (width 0.6) (layer "F.Cu") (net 17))
 (segment (start 129.54 91.44) (end 129.54 111.915662) (width 0.6) (layer "F.Cu") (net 17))
 (segment (start 111.76 126.05) (end 120.97 126.05) (width 0.6) (layer "B.Cu") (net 26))
 (segment (start 126.969338 127) (end 127.125 127.155662) (width 0.6) (layer "B.Cu") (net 26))
 (segment (start 120.97 126.05) (end 122.075662 127.155662) (width 0.6) (layer "B.Cu") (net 26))
 (segment (start 122.075662 127.155662) (end 127.125 127.155662) (width 0.6) (layer "B.Cu") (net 26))
 (segment (start 117.62 129.05) (end 118.11 129.54) (width 0.6) (layer "B.Cu") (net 7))
 (segment (start 117.8 68.58) (end 117.8 65.73) (width 0.6) (layer "B.Cu") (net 7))
 (segment (start 110.49 68.58) (end 110.49 87.59) (width 0.6) (layer "B.Cu") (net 7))
 (segment (start 114.3 64.77) (end 110.49 68.58) (width 0.6) (layer "B.Cu") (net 7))
 (segment (start 108.73 129.05) (end 111.76 129.05) (width 0.6) (layer "B.Cu") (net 7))
 (segment (start 153.5 128.720662) (end 153.5 126.55) (width 0.6) (layer "B.Cu") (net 7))
 (segment (start 117.8 65.73) (end 116.84 64.77) (width 0.6) (layer "B.Cu") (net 7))
 (segment (start 161.134338 94.135662) (end 161.29 93.98) (width 0.6) (layer "B.Cu") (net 7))
 (segment (start 118.11 129.54) (end 118.11 139.7) (width 0.6) (layer "B.Cu") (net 7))
 (segment (start 107.95 128.27) (end 108.73 129.05) (width 0.6) (layer "B.Cu") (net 7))
 (segment (start 107.99 93.385) (end 110.53 90.845) (width 0.6) (layer "B.Cu") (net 7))
 (segment (start 161.29 93.98) (end 161.29 77.47) (width 0.6) (layer "B.Cu") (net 7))
 (segment (start 149.985 94.135662) (end 161.134338 94.135662) (width 0.6) (layer "B.Cu") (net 7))
 (segment (start 111.76 129.05) (end 117.62 129.05) (width 0.6) (layer "B.Cu") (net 7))
 (segment (start 149.937306 94.183356) (end 149.985 94.135662) (width 0.6) (layer "B.Cu") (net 7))
 (segment (start 117.8 77.16) (end 117.8 68.58) (width 0.6) (layer "B.Cu") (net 7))
 (segment (start 134.62 105.41) (end 145.846644 94.183356) (width 0.6) (layer "B.Cu") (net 7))
 (segment (start 149.985 132.235662) (end 153.5 128.720662) (width 0.6) (layer "B.Cu") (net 7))
 (segment (start 107.95 94.02) (end 107.95 128.27) (width 0.6) (layer "B.Cu") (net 7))
 (segment (start 107.99 93.98) (end 107.99 93.385) (width 0.6) (layer "B.Cu") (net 7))
 (segment (start 118.11 139.7) (end 119.38 140.97) (width 0.6) (layer "B.Cu") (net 7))
 (segment (start 134.62 131.28) (end 134.62 105.41) (width 0.6) (layer "B.Cu") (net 7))
 (segment (start 127.72 138.18) (end 134.62 131.28) (width 0.6) (layer "B.Cu") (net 7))
 (segment (start 116.84 64.77) (end 114.3 64.77) (width 0.6) (layer "B.Cu") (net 7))
 (segment (start 107.99 93.98) (end 107.95 94.02) (width 0.6) (layer "B.Cu") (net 7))
 (segment (start 168 126.55) (end 168 100.69) (width 0.6) (layer "B.Cu") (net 7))
 (segment (start 149.985 132.235662) (end 149.985 140.97) (width 0.6) (layer "B.Cu") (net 7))
 (segment (start 110.53 90.845) (end 110.53 87.63) (width 0.6) (layer "B.Cu") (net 7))
 (segment (start 168 100.69) (end 161.29 93.98) (width 0.6) (layer "B.Cu") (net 7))
 (segment (start 153.035 77.47) (end 148.59 81.915) (width 0.6) (layer "B.Cu") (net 7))
 (segment (start 149.985 140.97) (end 119.38 140.97) (width 0.6) (layer "B.Cu") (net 7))
 (segment (start 161.29 77.47) (end 153.035 77.47) (width 0.6) (layer "B.Cu") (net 7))
 (segment (start 148.59 81.915) (end 122.555 81.915) (width 0.6) (layer "B.Cu") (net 7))
 (segment (start 145.846644 94.183356) (end 149.937306 94.183356) (width 0.6) (layer "B.Cu") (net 7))
 (segment (start 122.555 81.915) (end 117.8 77.16) (width 0.6) (layer "B.Cu") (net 7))
 (segment (start 110.49 87.59) (end 110.53 87.63) (width 0.6) (layer "B.Cu") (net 7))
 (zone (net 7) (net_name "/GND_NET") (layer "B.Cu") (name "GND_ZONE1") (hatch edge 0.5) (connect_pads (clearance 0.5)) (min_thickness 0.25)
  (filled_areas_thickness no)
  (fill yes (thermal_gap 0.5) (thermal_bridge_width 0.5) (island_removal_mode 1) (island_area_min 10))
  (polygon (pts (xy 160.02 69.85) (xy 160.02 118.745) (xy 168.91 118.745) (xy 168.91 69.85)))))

